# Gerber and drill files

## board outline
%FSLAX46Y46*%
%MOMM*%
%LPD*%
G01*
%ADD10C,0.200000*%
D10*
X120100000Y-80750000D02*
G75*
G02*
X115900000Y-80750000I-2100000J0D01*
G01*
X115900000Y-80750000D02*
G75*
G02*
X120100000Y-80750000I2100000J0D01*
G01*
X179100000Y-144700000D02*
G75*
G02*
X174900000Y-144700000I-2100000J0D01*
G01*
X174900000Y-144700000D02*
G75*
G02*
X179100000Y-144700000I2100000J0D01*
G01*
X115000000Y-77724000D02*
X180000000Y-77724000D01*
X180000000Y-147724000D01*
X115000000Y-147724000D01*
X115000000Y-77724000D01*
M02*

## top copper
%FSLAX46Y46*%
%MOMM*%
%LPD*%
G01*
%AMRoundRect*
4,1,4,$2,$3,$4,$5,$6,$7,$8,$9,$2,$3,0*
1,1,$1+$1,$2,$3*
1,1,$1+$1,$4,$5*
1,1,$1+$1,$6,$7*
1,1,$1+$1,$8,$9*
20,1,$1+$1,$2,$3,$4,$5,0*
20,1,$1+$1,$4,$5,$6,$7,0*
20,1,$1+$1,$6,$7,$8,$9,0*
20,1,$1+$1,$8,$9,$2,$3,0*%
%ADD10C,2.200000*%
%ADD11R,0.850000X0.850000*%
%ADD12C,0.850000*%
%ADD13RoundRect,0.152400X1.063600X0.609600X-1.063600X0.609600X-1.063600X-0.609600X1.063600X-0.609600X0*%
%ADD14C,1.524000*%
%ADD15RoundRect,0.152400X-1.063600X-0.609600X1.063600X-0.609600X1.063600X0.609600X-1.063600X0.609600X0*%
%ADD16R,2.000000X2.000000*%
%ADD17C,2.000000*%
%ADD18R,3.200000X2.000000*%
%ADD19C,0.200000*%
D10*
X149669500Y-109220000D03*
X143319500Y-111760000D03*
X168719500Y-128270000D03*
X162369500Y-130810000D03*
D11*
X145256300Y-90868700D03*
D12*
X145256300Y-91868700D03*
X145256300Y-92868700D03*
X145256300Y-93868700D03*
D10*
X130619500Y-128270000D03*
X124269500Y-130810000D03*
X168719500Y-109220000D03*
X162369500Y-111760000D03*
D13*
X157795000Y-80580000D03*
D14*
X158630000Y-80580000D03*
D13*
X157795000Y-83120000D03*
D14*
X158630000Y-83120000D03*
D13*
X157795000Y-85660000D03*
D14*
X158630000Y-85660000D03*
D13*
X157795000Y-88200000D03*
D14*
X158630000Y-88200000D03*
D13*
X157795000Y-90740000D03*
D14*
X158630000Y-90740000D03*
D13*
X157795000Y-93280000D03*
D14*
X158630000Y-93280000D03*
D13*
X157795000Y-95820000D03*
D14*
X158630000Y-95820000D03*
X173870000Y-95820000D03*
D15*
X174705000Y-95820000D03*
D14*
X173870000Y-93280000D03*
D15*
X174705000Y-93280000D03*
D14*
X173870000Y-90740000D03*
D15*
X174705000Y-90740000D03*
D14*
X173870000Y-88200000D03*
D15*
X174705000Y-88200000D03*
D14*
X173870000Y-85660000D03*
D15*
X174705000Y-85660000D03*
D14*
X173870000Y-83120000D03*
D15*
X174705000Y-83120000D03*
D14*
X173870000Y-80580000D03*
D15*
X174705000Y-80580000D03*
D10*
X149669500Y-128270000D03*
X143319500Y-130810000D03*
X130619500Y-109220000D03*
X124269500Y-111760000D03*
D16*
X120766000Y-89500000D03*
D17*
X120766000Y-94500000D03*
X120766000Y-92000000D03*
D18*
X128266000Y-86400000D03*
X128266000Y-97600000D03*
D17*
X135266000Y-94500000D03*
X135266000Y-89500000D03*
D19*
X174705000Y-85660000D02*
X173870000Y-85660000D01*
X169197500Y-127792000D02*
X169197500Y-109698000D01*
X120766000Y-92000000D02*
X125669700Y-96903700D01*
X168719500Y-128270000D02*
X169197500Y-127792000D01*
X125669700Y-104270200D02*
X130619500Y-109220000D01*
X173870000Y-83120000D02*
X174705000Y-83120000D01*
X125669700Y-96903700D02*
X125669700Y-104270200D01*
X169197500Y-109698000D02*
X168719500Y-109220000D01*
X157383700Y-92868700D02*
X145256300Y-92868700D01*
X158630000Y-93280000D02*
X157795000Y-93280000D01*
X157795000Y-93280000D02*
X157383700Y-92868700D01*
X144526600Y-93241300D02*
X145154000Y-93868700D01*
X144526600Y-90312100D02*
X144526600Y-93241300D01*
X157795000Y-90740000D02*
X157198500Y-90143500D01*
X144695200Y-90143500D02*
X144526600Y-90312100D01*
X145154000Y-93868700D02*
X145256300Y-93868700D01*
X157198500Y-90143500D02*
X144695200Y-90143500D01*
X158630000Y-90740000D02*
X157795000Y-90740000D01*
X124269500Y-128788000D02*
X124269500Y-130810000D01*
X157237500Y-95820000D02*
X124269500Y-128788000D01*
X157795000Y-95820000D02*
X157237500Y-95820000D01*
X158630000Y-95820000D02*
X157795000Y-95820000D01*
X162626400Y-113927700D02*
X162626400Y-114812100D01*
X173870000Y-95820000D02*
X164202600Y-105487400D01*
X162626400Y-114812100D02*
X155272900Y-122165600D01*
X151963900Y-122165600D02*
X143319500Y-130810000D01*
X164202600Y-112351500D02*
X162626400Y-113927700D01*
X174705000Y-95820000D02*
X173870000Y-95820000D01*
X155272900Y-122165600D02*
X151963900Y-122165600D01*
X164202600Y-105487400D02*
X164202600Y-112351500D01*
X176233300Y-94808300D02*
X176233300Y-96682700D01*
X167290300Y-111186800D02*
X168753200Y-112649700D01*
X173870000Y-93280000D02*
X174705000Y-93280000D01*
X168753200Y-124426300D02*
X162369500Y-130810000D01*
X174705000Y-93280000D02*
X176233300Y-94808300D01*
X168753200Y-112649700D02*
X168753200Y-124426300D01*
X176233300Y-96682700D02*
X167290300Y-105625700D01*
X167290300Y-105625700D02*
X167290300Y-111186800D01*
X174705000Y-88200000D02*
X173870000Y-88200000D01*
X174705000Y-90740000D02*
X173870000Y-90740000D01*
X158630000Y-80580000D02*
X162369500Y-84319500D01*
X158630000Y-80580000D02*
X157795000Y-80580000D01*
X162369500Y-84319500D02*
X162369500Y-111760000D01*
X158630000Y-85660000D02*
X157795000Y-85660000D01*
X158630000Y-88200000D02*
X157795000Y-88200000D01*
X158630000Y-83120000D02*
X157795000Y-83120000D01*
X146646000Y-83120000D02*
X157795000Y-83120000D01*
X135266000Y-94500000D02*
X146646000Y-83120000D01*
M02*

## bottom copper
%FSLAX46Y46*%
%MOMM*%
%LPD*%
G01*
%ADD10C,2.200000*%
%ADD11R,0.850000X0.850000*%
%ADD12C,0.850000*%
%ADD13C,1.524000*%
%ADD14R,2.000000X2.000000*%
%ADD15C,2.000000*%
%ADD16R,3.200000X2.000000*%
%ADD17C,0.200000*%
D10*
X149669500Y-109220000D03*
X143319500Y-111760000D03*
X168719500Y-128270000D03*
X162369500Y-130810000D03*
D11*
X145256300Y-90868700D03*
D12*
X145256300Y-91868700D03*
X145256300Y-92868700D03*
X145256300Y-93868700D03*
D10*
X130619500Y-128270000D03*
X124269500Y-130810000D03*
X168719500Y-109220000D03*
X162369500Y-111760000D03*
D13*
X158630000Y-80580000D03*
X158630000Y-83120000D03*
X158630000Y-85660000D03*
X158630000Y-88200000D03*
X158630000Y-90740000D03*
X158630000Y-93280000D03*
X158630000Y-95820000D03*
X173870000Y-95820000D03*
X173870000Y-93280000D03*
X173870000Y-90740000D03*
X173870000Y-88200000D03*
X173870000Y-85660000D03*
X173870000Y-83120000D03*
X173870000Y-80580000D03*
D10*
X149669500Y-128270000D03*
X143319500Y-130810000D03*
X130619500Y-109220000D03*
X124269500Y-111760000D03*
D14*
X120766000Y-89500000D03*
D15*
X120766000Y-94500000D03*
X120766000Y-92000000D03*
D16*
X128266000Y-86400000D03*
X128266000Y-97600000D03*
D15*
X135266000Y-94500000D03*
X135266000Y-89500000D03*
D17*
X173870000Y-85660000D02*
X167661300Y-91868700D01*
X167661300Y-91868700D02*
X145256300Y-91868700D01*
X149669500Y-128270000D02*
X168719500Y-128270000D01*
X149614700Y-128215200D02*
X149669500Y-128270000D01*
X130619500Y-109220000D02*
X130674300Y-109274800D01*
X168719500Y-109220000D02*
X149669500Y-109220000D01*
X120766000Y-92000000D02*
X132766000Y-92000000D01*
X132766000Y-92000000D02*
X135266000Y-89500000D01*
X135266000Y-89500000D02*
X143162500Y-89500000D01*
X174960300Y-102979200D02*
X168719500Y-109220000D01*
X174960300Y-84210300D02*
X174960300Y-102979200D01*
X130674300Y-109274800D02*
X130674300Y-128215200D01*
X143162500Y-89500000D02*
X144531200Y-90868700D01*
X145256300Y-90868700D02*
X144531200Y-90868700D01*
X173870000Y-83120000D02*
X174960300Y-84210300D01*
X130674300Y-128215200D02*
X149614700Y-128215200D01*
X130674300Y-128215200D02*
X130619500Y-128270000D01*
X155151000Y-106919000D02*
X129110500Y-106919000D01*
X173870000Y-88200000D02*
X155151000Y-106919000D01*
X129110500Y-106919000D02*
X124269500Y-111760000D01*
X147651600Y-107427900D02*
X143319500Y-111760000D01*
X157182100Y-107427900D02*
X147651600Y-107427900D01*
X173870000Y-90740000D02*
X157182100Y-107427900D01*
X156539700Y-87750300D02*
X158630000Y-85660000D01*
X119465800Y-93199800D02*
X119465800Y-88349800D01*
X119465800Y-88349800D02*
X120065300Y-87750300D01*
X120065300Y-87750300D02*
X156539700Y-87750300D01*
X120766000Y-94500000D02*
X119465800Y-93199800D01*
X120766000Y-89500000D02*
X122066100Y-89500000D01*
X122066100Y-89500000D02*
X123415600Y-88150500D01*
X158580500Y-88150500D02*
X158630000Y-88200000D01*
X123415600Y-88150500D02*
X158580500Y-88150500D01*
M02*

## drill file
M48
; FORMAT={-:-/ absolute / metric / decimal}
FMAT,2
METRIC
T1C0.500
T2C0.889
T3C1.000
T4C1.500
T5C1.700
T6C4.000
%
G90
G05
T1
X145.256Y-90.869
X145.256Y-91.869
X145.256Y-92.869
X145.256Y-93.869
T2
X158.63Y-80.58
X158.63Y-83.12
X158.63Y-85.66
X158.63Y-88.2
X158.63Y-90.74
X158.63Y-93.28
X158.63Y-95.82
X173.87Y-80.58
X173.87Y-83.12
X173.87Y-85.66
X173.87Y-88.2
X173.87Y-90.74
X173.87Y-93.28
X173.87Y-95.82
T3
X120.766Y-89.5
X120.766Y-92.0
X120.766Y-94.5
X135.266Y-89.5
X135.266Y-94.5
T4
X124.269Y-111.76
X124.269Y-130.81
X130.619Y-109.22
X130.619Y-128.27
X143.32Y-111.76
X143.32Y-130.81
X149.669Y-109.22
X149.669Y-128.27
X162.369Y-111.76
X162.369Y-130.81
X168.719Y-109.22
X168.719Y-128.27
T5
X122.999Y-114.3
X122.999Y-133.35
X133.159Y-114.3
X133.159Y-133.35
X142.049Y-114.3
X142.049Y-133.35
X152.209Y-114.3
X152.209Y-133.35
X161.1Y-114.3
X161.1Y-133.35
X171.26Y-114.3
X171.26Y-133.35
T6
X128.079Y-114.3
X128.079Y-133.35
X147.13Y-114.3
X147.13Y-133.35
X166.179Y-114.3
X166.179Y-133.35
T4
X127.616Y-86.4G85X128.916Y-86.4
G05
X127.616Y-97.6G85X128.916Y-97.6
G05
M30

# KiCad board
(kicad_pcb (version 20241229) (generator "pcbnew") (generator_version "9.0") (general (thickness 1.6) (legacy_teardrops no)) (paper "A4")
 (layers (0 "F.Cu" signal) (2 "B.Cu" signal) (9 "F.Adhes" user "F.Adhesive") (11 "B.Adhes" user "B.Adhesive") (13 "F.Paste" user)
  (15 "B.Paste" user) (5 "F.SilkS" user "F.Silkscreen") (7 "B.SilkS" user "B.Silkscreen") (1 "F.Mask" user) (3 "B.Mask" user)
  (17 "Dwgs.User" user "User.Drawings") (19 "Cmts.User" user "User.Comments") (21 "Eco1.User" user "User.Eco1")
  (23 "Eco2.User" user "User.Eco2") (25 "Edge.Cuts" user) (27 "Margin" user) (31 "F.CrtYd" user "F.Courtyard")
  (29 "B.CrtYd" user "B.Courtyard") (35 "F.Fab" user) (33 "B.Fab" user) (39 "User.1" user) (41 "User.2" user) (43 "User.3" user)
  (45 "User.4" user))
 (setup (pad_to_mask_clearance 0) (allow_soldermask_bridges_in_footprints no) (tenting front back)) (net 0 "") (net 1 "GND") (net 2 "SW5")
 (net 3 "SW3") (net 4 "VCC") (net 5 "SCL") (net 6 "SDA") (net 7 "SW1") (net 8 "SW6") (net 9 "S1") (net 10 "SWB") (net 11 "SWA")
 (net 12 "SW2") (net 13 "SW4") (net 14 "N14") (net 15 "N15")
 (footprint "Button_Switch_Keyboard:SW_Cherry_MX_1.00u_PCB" (layer "F.Cu") (at 149.6695 109.22)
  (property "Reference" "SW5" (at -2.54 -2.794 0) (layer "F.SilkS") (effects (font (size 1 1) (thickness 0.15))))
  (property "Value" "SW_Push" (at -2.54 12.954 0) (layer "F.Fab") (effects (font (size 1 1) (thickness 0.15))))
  (pad "" np_thru_hole circle (at -7.62 5.08) (size 1.7 1.7) (drill 1.7) (layers "*.Cu" "*.Mask"))
  (pad "" np_thru_hole circle (at -2.54 5.08) (size 4 4) (drill 4) (layers "*.Cu" "*.Mask"))
  (pad "" np_thru_hole circle (at 2.54 5.08) (size 1.7 1.7) (drill 1.7) (layers "*.Cu" "*.Mask"))
  (pad "1" thru_hole circle (at 0 0) (size 2.2 2.2) (drill 1.5) (layers "*.Cu" "*.Mask") (remove_unused_layers no) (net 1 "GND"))
  (pad "2" thru_hole circle (at -6.35 2.54) (size 2.2 2.2) (drill 1.5) (layers "*.Cu" "*.Mask") (remove_unused_layers no) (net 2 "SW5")))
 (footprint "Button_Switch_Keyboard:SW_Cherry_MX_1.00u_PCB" (layer "F.Cu") (at 168.7195 128.27)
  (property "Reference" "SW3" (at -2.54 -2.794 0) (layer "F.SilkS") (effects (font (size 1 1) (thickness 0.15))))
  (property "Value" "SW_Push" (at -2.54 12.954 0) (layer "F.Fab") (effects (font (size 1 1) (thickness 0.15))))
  (pad "" np_thru_hole circle (at -7.62 5.08) (size 1.7 1.7) (drill 1.7) (layers "*.Cu" "*.Mask"))
  (pad "" np_thru_hole circle (at -2.54 5.08) (size 4 4) (drill 4) (layers "*.Cu" "*.Mask"))
  (pad "" np_thru_hole circle (at 2.54 5.08) (size 1.7 1.7) (drill 1.7) (layers "*.Cu" "*.Mask"))
  (pad "1" thru_hole circle (at 0 0) (size 2.2 2.2) (drill 1.5) (layers "*.Cu" "*.Mask") (remove_unused_layers no) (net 1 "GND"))
  (pad "2" thru_hole circle (at -6.35 2.54) (size 2.2 2.2) (drill 1.5) (layers "*.Cu" "*.Mask") (remove_unused_layers no) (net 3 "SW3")))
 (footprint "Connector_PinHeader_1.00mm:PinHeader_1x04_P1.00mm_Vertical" (layer "F.Cu") (at 145.2563 90.8687)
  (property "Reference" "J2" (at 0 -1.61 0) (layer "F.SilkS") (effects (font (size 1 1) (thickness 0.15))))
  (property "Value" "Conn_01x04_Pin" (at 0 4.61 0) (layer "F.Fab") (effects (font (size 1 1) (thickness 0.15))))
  (pad "1" thru_hole rect (at 0 0) (size 0.85 0.85) (drill 0.5) (layers "*.Cu" "*.Mask") (remove_unused_layers no) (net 1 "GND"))
  (pad "2" thru_hole circle (at 0 1) (size 0.85 0.85) (drill 0.5) (layers "*.Cu" "*.Mask") (remove_unused_layers no) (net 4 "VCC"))
  (pad "3" thru_hole circle (at 0 2) (size 0.85 0.85) (drill 0.5) (layers "*.Cu" "*.Mask") (remove_unused_layers no) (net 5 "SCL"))
  (pad "4" thru_hole circle (at 0 3) (size 0.85 0.85) (drill 0.5) (layers "*.Cu" "*.Mask") (remove_unused_layers no) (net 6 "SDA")))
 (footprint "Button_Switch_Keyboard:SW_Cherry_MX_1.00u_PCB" (layer "F.Cu") (at 130.6195 128.27)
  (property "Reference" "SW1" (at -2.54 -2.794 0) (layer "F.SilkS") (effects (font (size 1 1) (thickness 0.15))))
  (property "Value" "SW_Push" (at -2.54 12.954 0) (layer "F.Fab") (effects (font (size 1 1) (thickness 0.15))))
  (pad "" np_thru_hole circle (at -7.62 5.08) (size 1.7 1.7) (drill 1.7) (layers "*.Cu" "*.Mask"))
  (pad "" np_thru_hole circle (at -2.54 5.08) (size 4 4) (drill 4) (layers "*.Cu" "*.Mask"))
  (pad "" np_thru_hole circle (at 2.54 5.08) (size 1.7 1.7) (drill 1.7) (layers "*.Cu" "*.Mask"))
  (pad "1" thru_hole circle (at 0 0) (size 2.2 2.2) (drill 1.5) (layers "*.Cu" "*.Mask") (remove_unused_layers no) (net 1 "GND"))
  (pad "2" thru_hole circle (at -6.35 2.54) (size 2.2 2.2) (drill 1.5) (layers "*.Cu" "*.Mask") (remove_unused_layers no) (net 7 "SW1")))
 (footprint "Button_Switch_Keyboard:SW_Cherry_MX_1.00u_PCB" (layer "F.Cu") (at 168.7195 109.22)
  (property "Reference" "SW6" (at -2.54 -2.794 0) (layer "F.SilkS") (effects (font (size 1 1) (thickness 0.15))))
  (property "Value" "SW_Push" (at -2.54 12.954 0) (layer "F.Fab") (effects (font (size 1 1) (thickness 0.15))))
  (pad "" np_thru_hole circle (at -7.62 5.08) (size 1.7 1.7) (drill 1.7) (layers "*.Cu" "*.Mask"))
  (pad "" np_thru_hole circle (at -2.54 5.08) (size 4 4) (drill 4) (layers "*.Cu" "*.Mask"))
  (pad "" np_thru_hole circle (at 2.54 5.08) (size 1.7 1.7) (drill 1.7) (layers "*.Cu" "*.Mask"))
  (pad "1" thru_hole circle (at 0 0) (size 2.2 2.2) (drill 1.5) (layers "*.Cu" "*.Mask") (remove_unused_layers no) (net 1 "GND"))
  (pad "2" thru_hole circle (at -6.35 2.54) (size 2.2 2.2) (drill 1.5) (layers "*.Cu" "*.Mask") (remove_unused_layers no) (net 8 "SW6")))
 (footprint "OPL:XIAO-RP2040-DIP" (layer "F.Cu") (at 166.25 88.2)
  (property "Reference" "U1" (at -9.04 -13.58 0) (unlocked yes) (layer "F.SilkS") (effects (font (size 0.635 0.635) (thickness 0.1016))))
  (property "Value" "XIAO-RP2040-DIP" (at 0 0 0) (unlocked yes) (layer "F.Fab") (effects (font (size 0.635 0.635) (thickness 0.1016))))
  (pad "1" smd roundrect (at -8.455 -7.62 180) (size 2.432 1.524) (layers "F.Cu" "F.Mask") (roundrect_rratio 0.1) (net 8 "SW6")
   (thermal_bridge_angle 45))
  (pad "1" thru_hole circle (at -7.62 -7.62 180) (size 1.524 1.524) (drill 0.889) (layers "*.Cu" "*.Mask") (remove_unused_layers no)
   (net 8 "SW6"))
  (pad "2" smd roundrect (at -8.455 -5.08 180) (size 2.432 1.524) (layers "F.Cu" "F.Mask") (roundrect_rratio 0.1) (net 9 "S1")
   (thermal_bridge_angle 45))
  (pad "2" thru_hole circle (at -7.62 -5.08 180) (size 1.524 1.524) (drill 0.889) (layers "*.Cu" "*.Mask") (remove_unused_layers no)
   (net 9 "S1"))
  (pad "3" smd roundrect (at -8.455 -2.54 180) (size 2.432 1.524) (layers "F.Cu" "F.Mask") (roundrect_rratio 0.1) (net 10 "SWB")
   (thermal_bridge_angle 45))
  (pad "3" thru_hole circle (at -7.62 -2.54 180) (size 1.524 1.524) (drill 0.889) (layers "*.Cu" "*.Mask") (remove_unused_layers no)
   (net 10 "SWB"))
  (pad "4" smd roundrect (at -8.455 0 180) (size 2.432 1.524) (layers "F.Cu" "F.Mask") (roundrect_rratio 0.1) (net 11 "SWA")
   (thermal_bridge_angle 45))
  (pad "4" thru_hole circle (at -7.62 0 180) (size 1.524 1.524) (drill 0.889) (layers "*.Cu" "*.Mask") (remove_unused_layers no)
   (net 11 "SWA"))
  (pad "5" smd roundrect (at -8.455 2.54 180) (size 2.432 1.524) (layers "F.Cu" "F.Mask") (roundrect_rratio 0.1) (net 6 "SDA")
   (thermal_bridge_angle 45))
  (pad "5" thru_hole circle (at -7.62 2.54 180) (size 1.524 1.524) (drill 0.889) (layers "*.Cu" "*.Mask") (remove_unused_layers no)
   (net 6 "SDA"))
  (pad "6" smd roundrect (at -8.455 5.08 180) (size 2.432 1.524) (layers "F.Cu" "F.Mask") (roundrect_rratio 0.1) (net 5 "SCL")
   (thermal_bridge_angle 45))
  (pad "6" thru_hole circle (at -7.62 5.08 180) (size 1.524 1.524) (drill 0.889) (layers "*.Cu" "*.Mask") (remove_unused_layers no)
   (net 5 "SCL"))
  (pad "7" smd roundrect (at -8.455 7.62 180) (size 2.432 1.524) (layers "F.Cu" "F.Mask") (roundrect_rratio 0.1) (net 7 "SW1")
   (thermal_bridge_angle 45))
  (pad "7" thru_hole circle (at -7.62 7.62 180) (size 1.524 1.524) (drill 0.889) (layers "*.Cu" "*.Mask") (remove_unused_layers no)
   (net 7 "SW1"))
  (pad "8" thru_hole circle (at 7.62 7.62) (size 1.524 1.524) (drill 0.889) (layers "*.Cu" "*.Mask") (remove_unused_layers no)
   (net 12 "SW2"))
  (pad "8" smd roundrect (at 8.455 7.62) (size 2.432 1.524) (layers "F.Cu" "F.Mask") (roundrect_rratio 0.1) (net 12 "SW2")
   (thermal_bridge_angle 45))
  (pad "9" thru_hole circle (at 7.62 5.08) (size 1.524 1.524) (drill 0.889) (layers "*.Cu" "*.Mask") (remove_unused_layers no) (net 3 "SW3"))
  (pad "9" smd roundrect (at 8.455 5.08) (size 2.432 1.524) (layers "F.Cu" "F.Mask") (roundrect_rratio 0.1) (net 3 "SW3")
   (thermal_bridge_angle 45))
  (pad "10" thru_hole circle (at 7.62 2.54) (size 1.524 1.524) (drill 0.889) (layers "*.Cu" "*.Mask") (remove_unused_layers no)
   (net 2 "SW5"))
  (pad "10" smd roundrect (at 8.455 2.54) (size 2.432 1.524) (layers "F.Cu" "F.Mask") (roundrect_rratio 0.1) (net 2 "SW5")
   (thermal_bridge_angle 45))
  (pad "11" thru_hole circle (at 7.62 0) (size 1.524 1.524) (drill 0.889) (layers "*.Cu" "*.Mask") (remove_unused_layers no) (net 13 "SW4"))
  (pad "11" smd roundrect (at 8.455 0) (size 2.432 1.524) (layers "F.Cu" "F.Mask") (roundrect_rratio 0.1) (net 13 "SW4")
   (thermal_bridge_angle 45))
  (pad "12" thru_hole circle (at 7.62 -2.54) (size 1.524 1.524) (drill 0.889) (layers "*.Cu" "*.Mask") (remove_unused_layers no)
   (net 4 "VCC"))
  (pad "12" smd roundrect (at 8.455 -2.54) (size 2.432 1.524) (layers "F.Cu" "F.Mask") (roundrect_rratio 0.1) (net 4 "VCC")
   (thermal_bridge_angle 45))
  (pad "13" thru_hole circle (at 7.62 -5.08) (size 1.524 1.524) (drill 0.889) (layers "*.Cu" "*.Mask") (remove_unused_layers no)
   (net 1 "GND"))
  (pad "13" smd roundrect (at 8.455 -5.08) (size 2.432 1.524) (layers "F.Cu" "F.Mask") (roundrect_rratio 0.1) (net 1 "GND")
   (thermal_bridge_angle 45))
  (pad "14" thru_hole circle (at 7.62 -7.62) (size 1.524 1.524) (drill 0.889) (layers "*.Cu" "*.Mask") (remove_unused_layers no)
   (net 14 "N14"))
  (pad "14" smd roundrect (at 8.455 -7.62) (size 2.432 1.524) (layers "F.Cu" "F.Mask") (roundrect_rratio 0.1) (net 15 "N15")
   (thermal_bridge_angle 45)))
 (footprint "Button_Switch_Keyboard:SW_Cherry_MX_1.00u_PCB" (layer "F.Cu") (at 149.6695 128.27)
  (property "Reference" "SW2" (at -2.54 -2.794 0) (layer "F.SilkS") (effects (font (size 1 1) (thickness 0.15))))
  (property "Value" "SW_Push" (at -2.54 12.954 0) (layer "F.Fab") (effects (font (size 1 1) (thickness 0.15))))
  (pad "" np_thru_hole circle (at -7.62 5.08) (size 1.7 1.7) (drill 1.7) (layers "*.Cu" "*.Mask"))
  (pad "" np_thru_hole circle (at -2.54 5.08) (size 4 4) (drill 4) (layers "*.Cu" "*.Mask"))
  (pad "" np_thru_hole circle (at 2.54 5.08) (size 1.7 1.7) (drill 1.7) (layers "*.Cu" "*.Mask"))
  (pad "1" thru_hole circle (at 0 0) (size 2.2 2.2) (drill 1.5) (layers "*.Cu" "*.Mask") (remove_unused_layers no) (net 1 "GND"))
  (pad "2" thru_hole circle (at -6.35 2.54) (size 2.2 2.2) (drill 1.5) (layers "*.Cu" "*.Mask") (remove_unused_layers no) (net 12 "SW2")))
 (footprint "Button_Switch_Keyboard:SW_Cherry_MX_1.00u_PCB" (layer "F.Cu") (at 130.6195 109.22)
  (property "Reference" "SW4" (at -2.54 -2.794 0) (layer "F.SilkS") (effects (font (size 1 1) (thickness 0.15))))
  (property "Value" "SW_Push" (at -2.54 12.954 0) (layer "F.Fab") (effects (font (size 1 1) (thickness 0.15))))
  (pad "" np_thru_hole circle (at -7.62 5.08) (size 1.7 1.7) (drill 1.7) (layers "*.Cu" "*.Mask"))
  (pad "" np_thru_hole circle (at -2.54 5.08) (size 4 4) (drill 4) (layers "*.Cu" "*.Mask"))
  (pad "" np_thru_hole circle (at 2.54 5.08) (size 1.7 1.7) (drill 1.7) (layers "*.Cu" "*.Mask"))
  (pad "1" thru_hole circle (at 0 0) (size 2.2 2.2) (drill 1.5) (layers "*.Cu" "*.Mask") (remove_unused_layers no) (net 1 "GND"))
  (pad "2" thru_hole circle (at -6.35 2.54) (size 2.2 2.2) (drill 1.5) (layers "*.Cu" "*.Mask") (remove_unused_layers no) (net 13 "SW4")))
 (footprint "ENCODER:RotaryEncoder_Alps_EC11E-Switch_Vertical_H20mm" (layer "F.Cu") (at 120.766 89.5)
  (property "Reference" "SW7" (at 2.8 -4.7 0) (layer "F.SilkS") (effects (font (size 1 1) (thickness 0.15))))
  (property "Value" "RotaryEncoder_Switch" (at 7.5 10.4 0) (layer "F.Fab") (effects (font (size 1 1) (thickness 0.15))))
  (pad "A" thru_hole rect (at 0 0) (size 2 2) (drill 1) (layers "*.Cu" "*.Mask") (remove_unused_layers no) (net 11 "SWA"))
  (pad "B" thru_hole circle (at 0 5) (size 2 2) (drill 1) (layers "*.Cu" "*.Mask") (remove_unused_layers no) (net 10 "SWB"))
  (pad "C" thru_hole circle (at 0 2.5) (size 2 2) (drill 1) (layers "*.Cu" "*.Mask") (remove_unused_layers no) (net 1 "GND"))
  (pad "MP" thru_hole rect (at 7.5 -3.1) (size 3.2 2) (drill oval 2.8 1.5) (layers "*.Cu" "*.Mask") (remove_unused_layers no))
  (pad "MP" thru_hole rect (at 7.5 8.1) (size 3.2 2) (drill oval 2.8 1.5) (layers "*.Cu" "*.Mask") (remove_unused_layers no))
  (pad "S1" thru_hole circle (at 14.5 5) (size 2 2) (drill 1) (layers "*.Cu" "*.Mask") (remove_unused_layers no) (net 9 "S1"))
  (pad "S2" thru_hole circle (at 14.5 0) (size 2 2) (drill 1) (layers "*.Cu" "*.Mask") (remove_unused_layers no) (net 1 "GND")))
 (gr_circle (center 118 80.75) (end 120.1 80.75) (stroke (width 0.2) (type solid)) (fill no) (layer "Edge.Cuts"))
 (gr_circle (center 177 144.7) (end 179.1 144.7) (stroke (width 0.2) (type solid)) (fill no) (layer "Edge.Cuts"))
 (gr_rect (start 115 77.724) (end 180 147.724) (stroke (width 0.2) (type solid)) (fill no) (layer "Edge.Cuts"))
 (segment (start 174.705 85.66) (end 173.87 85.66) (width 0.2) (layer "F.Cu") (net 4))
 (segment (start 173.87 85.66) (end 167.6613 91.8687) (width 0.2) (layer "B.Cu") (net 4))
 (segment (start 167.6613 91.8687) (end 145.2563 91.8687) (width 0.2) (layer "B.Cu") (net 4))
 (segment (start 169.1975 127.792) (end 169.1975 109.698) (width 0.2) (layer "F.Cu") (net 1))
 (segment (start 120.766 92) (end 125.6697 96.9037) (width 0.2) (layer "F.Cu") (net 1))
 (segment (start 168.7195 128.27) (end 169.1975 127.792) (width 0.2) (layer "F.Cu") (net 1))
 (segment (start 125.6697 104.2702) (end 130.6195 109.22) (width 0.2) (layer "F.Cu") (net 1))
 (segment (start 173.87 83.12) (end 174.705 83.12) (width 0.2) (layer "F.Cu") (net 1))
 (segment (start 125.6697 96.9037) (end 125.6697 104.2702) (width 0.2) (layer "F.Cu") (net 1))
 (segment (start 169.1975 109.698) (end 168.7195 109.22) (width 0.2) (layer "F.Cu") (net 1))
 (segment (start 149.6695 128.27) (end 168.7195 128.27) (width 0.2) (layer "B.Cu") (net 1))
 (segment (start 149.6147 128.2152) (end 149.6695 128.27) (width 0.2) (layer "B.Cu") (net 1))
 (segment (start 130.6195 109.22) (end 130.6743 109.2748) (width 0.2) (layer "B.Cu") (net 1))
 (segment (start 168.7195 109.22) (end 149.6695 109.22) (width 0.2) (layer "B.Cu") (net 1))
 (segment (start 120.766 92) (end 132.766 92) (width 0.2) (layer "B.Cu") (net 1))
 (segment (start 132.766 92) (end 135.266 89.5) (width 0.2) (layer "B.Cu") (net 1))
 (segment (start 135.266 89.5) (end 143.1625 89.5) (width 0.2) (layer "B.Cu") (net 1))
 (segment (start 174.9603 102.9792) (end 168.7195 109.22) (width 0.2) (layer "B.Cu") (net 1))
 (segment (start 174.9603 84.2103) (end 174.9603 102.9792) (width 0.2) (layer "B.Cu") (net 1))
 (segment (start 130.6743 109.2748) (end 130.6743 128.2152) (width 0.2) (layer "B.Cu") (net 1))
 (segment (start 143.1625 89.5) (end 144.5312 90.8687) (width 0.2) (layer "B.Cu") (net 1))
 (segment (start 145.2563 90.8687) (end 144.5312 90.8687) (width 0.2) (layer "B.Cu") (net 1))
 (segment (start 173.87 83.12) (end 174.9603 84.2103) (width 0.2) (layer "B.Cu") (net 1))
 (segment (start 130.6743 128.2152) (end 149.6147 128.2152) (width 0.2) (layer "B.Cu") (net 1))
 (segment (start 130.6743 128.2152) (end 130.6195 128.27) (width 0.2) (layer "B.Cu") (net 1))
 (segment (start 157.3837 92.8687) (end 145.2563 92.8687) (width 0.2) (layer "F.Cu") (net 5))
 (segment (start 158.63 93.28) (end 157.795 93.28) (width 0.2) (layer "F.Cu") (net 5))
 (segment (start 157.795 93.28) (end 157.3837 92.8687) (width 0.2) (layer "F.Cu") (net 5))
 (segment (start 144.5266 93.2413) (end 145.154 93.8687) (width 0.2) (layer "F.Cu") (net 6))
 (segment (start 144.5266 90.3121) (end 144.5266 93.2413) (width 0.2) (layer "F.Cu") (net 6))
 (segment (start 157.795 90.74) (end 157.1985 90.1435) (width 0.2) (layer "F.Cu") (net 6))
 (segment (start 144.6952 90.1435) (end 144.5266 90.3121) (width 0.2) (layer "F.Cu") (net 6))
 (segment (start 145.154 93.8687) (end 145.2563 93.8687) (width 0.2) (layer "F.Cu") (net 6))
 (segment (start 157.1985 90.1435) (end 144.6952 90.1435) (width 0.2) (layer "F.Cu") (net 6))
 (segment (start 158.63 90.74) (end 157.795 90.74) (width 0.2) (layer "F.Cu") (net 6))
 (segment (start 124.2695 128.788) (end 124.2695 130.81) (width 0.2) (layer "F.Cu") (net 7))
 (segment (start 157.2375 95.82) (end 124.2695 128.788) (width 0.2) (layer "F.Cu") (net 7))
 (segment (start 157.795 95.82) (end 157.2375 95.82) (width 0.2) (layer "F.Cu") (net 7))
 (segment (start 158.63 95.82) (end 157.795 95.82) (width 0.2) (layer "F.Cu") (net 7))
 (segment (start 162.6264 113.9277) (end 162.6264 114.8121) (width 0.2) (layer "F.Cu") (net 12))
 (segment (start 173.87 95.82) (end 164.2026 105.4874) (width 0.2) (layer "F.Cu") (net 12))
 (segment (start 162.6264 114.8121) (end 155.2729 122.1656) (width 0.2) (layer "F.Cu") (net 12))
 (segment (start 151.9639 122.1656) (end 143.3195 130.81) (width 0.2) (layer "F.Cu") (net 12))
 (segment (start 164.2026 112.3515) (end 162.6264 113.9277) (width 0.2) (layer "F.Cu") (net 12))
 (segment (start 174.705 95.82) (end 173.87 95.82) (width 0.2) (layer "F.Cu") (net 12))
 (segment (start 155.2729 122.1656) (end 151.9639 122.1656) (width 0.2) (layer "F.Cu") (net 12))
 (segment (start 164.2026 105.4874) (end 164.2026 112.3515) (width 0.2) (layer "F.Cu") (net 12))
 (segment (start 176.2333 94.8083) (end 176.2333 96.6827) (width 0.2) (layer "F.Cu") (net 3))
 (segment (start 167.2903 111.1868) (end 168.7532 112.6497) (width 0.2) (layer "F.Cu") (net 3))
 (segment (start 173.87 93.28) (end 174.705 93.28) (width 0.2) (layer "F.Cu") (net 3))
 (segment (start 168.7532 124.4263) (end 162.3695 130.81) (width 0.2) (layer "F.Cu") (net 3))
 (segment (start 174.705 93.28) (end 176.2333 94.8083) (width 0.2) (layer "F.Cu") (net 3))
 (segment (start 168.7532 112.6497) (end 168.7532 124.4263) (width 0.2) (layer "F.Cu") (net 3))
 (segment (start 176.2333 96.6827) (end 167.2903 105.6257) (width 0.2) (layer "F.Cu") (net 3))
 (segment (start 167.2903 105.6257) (end 167.2903 111.1868) (width 0.2) (layer "F.Cu") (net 3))
 (segment (start 174.705 88.2) (end 173.87 88.2) (width 0.2) (layer "F.Cu") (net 13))
 (segment (start 155.151 106.919) (end 129.1105 106.919) (width 0.2) (layer "B.Cu") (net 13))
 (segment (start 173.87 88.2) (end 155.151 106.919) (width 0.2) (layer "B.Cu") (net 13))
 (segment (start 129.1105 106.919) (end 124.2695 111.76) (width 0.2) (layer "B.Cu") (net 13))
 (segment (start 174.705 90.74) (end 173.87 90.74) (width 0.2) (layer "F.Cu") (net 2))
 (segment (start 147.6516 107.4279) (end 143.3195 111.76) (width 0.2) (layer "B.Cu") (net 2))
 (segment (start 157.1821 107.4279) (end 147.6516 107.4279) (width 0.2) (layer "B.Cu") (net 2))
 (segment (start 173.87 90.74) (end 157.1821 107.4279) (width 0.2) (layer "B.Cu") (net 2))
 (segment (start 158.63 80.58) (end 162.3695 84.3195) (width 0.2) (layer "F.Cu") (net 8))
 (segment (start 158.63 80.58) (end 157.795 80.58) (width 0.2) (layer "F.Cu") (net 8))
 (segment (start 162.3695 84.3195) (end 162.3695 111.76) (width 0.2) (layer "F.Cu") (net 8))
 (segment (start 158.63 85.66) (end 157.795 85.66) (width 0.2) (layer "F.Cu") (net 10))
 (segment (start 156.5397 87.7503) (end 158.63 85.66) (width 0.2) (layer "B.Cu") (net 10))
 (segment (start 119.4658 93.1998) (end 119.4658 88.3498) (width 0.2) (layer "B.Cu") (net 10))
 (segment (start 119.4658 88.3498) (end 120.0653 87.7503) (width 0.2) (layer "B.Cu") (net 10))
 (segment (start 120.0653 87.7503) (end 156.5397 87.7503) (width 0.2) (layer "B.Cu") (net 10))
 (segment (start 120.766 94.5) (end 119.4658 93.1998) (width 0.2) (layer "B.Cu") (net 10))
 (segment (start 158.63 88.2) (end 157.795 88.2) (width 0.2) (layer "F.Cu") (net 11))
 (segment (start 120.766 89.5) (end 122.0661 89.5) (width 0.2) (layer "B.Cu") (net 11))
 (segment (start 122.0661 89.5) (end 123.4156 88.1505) (width 0.2) (layer "B.Cu") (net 11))
 (segment (start 158.5805 88.1505) (end 158.63 88.2) (width 0.2) (layer "B.Cu") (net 11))
 (segment (start 123.4156 88.1505) (end 158.5805 88.1505) (width 0.2) (layer "B.Cu") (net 11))
 (segment (start 158.63 83.12) (end 157.795 83.12) (width 0.2) (layer "F.Cu") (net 9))
 (segment (start 146.646 83.12) (end 157.795 83.12) (width 0.2) (layer "F.Cu") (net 9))
 (segment (start 135.266 94.5) (end 146.646 83.12) (width 0.2) (layer "F.Cu") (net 9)))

